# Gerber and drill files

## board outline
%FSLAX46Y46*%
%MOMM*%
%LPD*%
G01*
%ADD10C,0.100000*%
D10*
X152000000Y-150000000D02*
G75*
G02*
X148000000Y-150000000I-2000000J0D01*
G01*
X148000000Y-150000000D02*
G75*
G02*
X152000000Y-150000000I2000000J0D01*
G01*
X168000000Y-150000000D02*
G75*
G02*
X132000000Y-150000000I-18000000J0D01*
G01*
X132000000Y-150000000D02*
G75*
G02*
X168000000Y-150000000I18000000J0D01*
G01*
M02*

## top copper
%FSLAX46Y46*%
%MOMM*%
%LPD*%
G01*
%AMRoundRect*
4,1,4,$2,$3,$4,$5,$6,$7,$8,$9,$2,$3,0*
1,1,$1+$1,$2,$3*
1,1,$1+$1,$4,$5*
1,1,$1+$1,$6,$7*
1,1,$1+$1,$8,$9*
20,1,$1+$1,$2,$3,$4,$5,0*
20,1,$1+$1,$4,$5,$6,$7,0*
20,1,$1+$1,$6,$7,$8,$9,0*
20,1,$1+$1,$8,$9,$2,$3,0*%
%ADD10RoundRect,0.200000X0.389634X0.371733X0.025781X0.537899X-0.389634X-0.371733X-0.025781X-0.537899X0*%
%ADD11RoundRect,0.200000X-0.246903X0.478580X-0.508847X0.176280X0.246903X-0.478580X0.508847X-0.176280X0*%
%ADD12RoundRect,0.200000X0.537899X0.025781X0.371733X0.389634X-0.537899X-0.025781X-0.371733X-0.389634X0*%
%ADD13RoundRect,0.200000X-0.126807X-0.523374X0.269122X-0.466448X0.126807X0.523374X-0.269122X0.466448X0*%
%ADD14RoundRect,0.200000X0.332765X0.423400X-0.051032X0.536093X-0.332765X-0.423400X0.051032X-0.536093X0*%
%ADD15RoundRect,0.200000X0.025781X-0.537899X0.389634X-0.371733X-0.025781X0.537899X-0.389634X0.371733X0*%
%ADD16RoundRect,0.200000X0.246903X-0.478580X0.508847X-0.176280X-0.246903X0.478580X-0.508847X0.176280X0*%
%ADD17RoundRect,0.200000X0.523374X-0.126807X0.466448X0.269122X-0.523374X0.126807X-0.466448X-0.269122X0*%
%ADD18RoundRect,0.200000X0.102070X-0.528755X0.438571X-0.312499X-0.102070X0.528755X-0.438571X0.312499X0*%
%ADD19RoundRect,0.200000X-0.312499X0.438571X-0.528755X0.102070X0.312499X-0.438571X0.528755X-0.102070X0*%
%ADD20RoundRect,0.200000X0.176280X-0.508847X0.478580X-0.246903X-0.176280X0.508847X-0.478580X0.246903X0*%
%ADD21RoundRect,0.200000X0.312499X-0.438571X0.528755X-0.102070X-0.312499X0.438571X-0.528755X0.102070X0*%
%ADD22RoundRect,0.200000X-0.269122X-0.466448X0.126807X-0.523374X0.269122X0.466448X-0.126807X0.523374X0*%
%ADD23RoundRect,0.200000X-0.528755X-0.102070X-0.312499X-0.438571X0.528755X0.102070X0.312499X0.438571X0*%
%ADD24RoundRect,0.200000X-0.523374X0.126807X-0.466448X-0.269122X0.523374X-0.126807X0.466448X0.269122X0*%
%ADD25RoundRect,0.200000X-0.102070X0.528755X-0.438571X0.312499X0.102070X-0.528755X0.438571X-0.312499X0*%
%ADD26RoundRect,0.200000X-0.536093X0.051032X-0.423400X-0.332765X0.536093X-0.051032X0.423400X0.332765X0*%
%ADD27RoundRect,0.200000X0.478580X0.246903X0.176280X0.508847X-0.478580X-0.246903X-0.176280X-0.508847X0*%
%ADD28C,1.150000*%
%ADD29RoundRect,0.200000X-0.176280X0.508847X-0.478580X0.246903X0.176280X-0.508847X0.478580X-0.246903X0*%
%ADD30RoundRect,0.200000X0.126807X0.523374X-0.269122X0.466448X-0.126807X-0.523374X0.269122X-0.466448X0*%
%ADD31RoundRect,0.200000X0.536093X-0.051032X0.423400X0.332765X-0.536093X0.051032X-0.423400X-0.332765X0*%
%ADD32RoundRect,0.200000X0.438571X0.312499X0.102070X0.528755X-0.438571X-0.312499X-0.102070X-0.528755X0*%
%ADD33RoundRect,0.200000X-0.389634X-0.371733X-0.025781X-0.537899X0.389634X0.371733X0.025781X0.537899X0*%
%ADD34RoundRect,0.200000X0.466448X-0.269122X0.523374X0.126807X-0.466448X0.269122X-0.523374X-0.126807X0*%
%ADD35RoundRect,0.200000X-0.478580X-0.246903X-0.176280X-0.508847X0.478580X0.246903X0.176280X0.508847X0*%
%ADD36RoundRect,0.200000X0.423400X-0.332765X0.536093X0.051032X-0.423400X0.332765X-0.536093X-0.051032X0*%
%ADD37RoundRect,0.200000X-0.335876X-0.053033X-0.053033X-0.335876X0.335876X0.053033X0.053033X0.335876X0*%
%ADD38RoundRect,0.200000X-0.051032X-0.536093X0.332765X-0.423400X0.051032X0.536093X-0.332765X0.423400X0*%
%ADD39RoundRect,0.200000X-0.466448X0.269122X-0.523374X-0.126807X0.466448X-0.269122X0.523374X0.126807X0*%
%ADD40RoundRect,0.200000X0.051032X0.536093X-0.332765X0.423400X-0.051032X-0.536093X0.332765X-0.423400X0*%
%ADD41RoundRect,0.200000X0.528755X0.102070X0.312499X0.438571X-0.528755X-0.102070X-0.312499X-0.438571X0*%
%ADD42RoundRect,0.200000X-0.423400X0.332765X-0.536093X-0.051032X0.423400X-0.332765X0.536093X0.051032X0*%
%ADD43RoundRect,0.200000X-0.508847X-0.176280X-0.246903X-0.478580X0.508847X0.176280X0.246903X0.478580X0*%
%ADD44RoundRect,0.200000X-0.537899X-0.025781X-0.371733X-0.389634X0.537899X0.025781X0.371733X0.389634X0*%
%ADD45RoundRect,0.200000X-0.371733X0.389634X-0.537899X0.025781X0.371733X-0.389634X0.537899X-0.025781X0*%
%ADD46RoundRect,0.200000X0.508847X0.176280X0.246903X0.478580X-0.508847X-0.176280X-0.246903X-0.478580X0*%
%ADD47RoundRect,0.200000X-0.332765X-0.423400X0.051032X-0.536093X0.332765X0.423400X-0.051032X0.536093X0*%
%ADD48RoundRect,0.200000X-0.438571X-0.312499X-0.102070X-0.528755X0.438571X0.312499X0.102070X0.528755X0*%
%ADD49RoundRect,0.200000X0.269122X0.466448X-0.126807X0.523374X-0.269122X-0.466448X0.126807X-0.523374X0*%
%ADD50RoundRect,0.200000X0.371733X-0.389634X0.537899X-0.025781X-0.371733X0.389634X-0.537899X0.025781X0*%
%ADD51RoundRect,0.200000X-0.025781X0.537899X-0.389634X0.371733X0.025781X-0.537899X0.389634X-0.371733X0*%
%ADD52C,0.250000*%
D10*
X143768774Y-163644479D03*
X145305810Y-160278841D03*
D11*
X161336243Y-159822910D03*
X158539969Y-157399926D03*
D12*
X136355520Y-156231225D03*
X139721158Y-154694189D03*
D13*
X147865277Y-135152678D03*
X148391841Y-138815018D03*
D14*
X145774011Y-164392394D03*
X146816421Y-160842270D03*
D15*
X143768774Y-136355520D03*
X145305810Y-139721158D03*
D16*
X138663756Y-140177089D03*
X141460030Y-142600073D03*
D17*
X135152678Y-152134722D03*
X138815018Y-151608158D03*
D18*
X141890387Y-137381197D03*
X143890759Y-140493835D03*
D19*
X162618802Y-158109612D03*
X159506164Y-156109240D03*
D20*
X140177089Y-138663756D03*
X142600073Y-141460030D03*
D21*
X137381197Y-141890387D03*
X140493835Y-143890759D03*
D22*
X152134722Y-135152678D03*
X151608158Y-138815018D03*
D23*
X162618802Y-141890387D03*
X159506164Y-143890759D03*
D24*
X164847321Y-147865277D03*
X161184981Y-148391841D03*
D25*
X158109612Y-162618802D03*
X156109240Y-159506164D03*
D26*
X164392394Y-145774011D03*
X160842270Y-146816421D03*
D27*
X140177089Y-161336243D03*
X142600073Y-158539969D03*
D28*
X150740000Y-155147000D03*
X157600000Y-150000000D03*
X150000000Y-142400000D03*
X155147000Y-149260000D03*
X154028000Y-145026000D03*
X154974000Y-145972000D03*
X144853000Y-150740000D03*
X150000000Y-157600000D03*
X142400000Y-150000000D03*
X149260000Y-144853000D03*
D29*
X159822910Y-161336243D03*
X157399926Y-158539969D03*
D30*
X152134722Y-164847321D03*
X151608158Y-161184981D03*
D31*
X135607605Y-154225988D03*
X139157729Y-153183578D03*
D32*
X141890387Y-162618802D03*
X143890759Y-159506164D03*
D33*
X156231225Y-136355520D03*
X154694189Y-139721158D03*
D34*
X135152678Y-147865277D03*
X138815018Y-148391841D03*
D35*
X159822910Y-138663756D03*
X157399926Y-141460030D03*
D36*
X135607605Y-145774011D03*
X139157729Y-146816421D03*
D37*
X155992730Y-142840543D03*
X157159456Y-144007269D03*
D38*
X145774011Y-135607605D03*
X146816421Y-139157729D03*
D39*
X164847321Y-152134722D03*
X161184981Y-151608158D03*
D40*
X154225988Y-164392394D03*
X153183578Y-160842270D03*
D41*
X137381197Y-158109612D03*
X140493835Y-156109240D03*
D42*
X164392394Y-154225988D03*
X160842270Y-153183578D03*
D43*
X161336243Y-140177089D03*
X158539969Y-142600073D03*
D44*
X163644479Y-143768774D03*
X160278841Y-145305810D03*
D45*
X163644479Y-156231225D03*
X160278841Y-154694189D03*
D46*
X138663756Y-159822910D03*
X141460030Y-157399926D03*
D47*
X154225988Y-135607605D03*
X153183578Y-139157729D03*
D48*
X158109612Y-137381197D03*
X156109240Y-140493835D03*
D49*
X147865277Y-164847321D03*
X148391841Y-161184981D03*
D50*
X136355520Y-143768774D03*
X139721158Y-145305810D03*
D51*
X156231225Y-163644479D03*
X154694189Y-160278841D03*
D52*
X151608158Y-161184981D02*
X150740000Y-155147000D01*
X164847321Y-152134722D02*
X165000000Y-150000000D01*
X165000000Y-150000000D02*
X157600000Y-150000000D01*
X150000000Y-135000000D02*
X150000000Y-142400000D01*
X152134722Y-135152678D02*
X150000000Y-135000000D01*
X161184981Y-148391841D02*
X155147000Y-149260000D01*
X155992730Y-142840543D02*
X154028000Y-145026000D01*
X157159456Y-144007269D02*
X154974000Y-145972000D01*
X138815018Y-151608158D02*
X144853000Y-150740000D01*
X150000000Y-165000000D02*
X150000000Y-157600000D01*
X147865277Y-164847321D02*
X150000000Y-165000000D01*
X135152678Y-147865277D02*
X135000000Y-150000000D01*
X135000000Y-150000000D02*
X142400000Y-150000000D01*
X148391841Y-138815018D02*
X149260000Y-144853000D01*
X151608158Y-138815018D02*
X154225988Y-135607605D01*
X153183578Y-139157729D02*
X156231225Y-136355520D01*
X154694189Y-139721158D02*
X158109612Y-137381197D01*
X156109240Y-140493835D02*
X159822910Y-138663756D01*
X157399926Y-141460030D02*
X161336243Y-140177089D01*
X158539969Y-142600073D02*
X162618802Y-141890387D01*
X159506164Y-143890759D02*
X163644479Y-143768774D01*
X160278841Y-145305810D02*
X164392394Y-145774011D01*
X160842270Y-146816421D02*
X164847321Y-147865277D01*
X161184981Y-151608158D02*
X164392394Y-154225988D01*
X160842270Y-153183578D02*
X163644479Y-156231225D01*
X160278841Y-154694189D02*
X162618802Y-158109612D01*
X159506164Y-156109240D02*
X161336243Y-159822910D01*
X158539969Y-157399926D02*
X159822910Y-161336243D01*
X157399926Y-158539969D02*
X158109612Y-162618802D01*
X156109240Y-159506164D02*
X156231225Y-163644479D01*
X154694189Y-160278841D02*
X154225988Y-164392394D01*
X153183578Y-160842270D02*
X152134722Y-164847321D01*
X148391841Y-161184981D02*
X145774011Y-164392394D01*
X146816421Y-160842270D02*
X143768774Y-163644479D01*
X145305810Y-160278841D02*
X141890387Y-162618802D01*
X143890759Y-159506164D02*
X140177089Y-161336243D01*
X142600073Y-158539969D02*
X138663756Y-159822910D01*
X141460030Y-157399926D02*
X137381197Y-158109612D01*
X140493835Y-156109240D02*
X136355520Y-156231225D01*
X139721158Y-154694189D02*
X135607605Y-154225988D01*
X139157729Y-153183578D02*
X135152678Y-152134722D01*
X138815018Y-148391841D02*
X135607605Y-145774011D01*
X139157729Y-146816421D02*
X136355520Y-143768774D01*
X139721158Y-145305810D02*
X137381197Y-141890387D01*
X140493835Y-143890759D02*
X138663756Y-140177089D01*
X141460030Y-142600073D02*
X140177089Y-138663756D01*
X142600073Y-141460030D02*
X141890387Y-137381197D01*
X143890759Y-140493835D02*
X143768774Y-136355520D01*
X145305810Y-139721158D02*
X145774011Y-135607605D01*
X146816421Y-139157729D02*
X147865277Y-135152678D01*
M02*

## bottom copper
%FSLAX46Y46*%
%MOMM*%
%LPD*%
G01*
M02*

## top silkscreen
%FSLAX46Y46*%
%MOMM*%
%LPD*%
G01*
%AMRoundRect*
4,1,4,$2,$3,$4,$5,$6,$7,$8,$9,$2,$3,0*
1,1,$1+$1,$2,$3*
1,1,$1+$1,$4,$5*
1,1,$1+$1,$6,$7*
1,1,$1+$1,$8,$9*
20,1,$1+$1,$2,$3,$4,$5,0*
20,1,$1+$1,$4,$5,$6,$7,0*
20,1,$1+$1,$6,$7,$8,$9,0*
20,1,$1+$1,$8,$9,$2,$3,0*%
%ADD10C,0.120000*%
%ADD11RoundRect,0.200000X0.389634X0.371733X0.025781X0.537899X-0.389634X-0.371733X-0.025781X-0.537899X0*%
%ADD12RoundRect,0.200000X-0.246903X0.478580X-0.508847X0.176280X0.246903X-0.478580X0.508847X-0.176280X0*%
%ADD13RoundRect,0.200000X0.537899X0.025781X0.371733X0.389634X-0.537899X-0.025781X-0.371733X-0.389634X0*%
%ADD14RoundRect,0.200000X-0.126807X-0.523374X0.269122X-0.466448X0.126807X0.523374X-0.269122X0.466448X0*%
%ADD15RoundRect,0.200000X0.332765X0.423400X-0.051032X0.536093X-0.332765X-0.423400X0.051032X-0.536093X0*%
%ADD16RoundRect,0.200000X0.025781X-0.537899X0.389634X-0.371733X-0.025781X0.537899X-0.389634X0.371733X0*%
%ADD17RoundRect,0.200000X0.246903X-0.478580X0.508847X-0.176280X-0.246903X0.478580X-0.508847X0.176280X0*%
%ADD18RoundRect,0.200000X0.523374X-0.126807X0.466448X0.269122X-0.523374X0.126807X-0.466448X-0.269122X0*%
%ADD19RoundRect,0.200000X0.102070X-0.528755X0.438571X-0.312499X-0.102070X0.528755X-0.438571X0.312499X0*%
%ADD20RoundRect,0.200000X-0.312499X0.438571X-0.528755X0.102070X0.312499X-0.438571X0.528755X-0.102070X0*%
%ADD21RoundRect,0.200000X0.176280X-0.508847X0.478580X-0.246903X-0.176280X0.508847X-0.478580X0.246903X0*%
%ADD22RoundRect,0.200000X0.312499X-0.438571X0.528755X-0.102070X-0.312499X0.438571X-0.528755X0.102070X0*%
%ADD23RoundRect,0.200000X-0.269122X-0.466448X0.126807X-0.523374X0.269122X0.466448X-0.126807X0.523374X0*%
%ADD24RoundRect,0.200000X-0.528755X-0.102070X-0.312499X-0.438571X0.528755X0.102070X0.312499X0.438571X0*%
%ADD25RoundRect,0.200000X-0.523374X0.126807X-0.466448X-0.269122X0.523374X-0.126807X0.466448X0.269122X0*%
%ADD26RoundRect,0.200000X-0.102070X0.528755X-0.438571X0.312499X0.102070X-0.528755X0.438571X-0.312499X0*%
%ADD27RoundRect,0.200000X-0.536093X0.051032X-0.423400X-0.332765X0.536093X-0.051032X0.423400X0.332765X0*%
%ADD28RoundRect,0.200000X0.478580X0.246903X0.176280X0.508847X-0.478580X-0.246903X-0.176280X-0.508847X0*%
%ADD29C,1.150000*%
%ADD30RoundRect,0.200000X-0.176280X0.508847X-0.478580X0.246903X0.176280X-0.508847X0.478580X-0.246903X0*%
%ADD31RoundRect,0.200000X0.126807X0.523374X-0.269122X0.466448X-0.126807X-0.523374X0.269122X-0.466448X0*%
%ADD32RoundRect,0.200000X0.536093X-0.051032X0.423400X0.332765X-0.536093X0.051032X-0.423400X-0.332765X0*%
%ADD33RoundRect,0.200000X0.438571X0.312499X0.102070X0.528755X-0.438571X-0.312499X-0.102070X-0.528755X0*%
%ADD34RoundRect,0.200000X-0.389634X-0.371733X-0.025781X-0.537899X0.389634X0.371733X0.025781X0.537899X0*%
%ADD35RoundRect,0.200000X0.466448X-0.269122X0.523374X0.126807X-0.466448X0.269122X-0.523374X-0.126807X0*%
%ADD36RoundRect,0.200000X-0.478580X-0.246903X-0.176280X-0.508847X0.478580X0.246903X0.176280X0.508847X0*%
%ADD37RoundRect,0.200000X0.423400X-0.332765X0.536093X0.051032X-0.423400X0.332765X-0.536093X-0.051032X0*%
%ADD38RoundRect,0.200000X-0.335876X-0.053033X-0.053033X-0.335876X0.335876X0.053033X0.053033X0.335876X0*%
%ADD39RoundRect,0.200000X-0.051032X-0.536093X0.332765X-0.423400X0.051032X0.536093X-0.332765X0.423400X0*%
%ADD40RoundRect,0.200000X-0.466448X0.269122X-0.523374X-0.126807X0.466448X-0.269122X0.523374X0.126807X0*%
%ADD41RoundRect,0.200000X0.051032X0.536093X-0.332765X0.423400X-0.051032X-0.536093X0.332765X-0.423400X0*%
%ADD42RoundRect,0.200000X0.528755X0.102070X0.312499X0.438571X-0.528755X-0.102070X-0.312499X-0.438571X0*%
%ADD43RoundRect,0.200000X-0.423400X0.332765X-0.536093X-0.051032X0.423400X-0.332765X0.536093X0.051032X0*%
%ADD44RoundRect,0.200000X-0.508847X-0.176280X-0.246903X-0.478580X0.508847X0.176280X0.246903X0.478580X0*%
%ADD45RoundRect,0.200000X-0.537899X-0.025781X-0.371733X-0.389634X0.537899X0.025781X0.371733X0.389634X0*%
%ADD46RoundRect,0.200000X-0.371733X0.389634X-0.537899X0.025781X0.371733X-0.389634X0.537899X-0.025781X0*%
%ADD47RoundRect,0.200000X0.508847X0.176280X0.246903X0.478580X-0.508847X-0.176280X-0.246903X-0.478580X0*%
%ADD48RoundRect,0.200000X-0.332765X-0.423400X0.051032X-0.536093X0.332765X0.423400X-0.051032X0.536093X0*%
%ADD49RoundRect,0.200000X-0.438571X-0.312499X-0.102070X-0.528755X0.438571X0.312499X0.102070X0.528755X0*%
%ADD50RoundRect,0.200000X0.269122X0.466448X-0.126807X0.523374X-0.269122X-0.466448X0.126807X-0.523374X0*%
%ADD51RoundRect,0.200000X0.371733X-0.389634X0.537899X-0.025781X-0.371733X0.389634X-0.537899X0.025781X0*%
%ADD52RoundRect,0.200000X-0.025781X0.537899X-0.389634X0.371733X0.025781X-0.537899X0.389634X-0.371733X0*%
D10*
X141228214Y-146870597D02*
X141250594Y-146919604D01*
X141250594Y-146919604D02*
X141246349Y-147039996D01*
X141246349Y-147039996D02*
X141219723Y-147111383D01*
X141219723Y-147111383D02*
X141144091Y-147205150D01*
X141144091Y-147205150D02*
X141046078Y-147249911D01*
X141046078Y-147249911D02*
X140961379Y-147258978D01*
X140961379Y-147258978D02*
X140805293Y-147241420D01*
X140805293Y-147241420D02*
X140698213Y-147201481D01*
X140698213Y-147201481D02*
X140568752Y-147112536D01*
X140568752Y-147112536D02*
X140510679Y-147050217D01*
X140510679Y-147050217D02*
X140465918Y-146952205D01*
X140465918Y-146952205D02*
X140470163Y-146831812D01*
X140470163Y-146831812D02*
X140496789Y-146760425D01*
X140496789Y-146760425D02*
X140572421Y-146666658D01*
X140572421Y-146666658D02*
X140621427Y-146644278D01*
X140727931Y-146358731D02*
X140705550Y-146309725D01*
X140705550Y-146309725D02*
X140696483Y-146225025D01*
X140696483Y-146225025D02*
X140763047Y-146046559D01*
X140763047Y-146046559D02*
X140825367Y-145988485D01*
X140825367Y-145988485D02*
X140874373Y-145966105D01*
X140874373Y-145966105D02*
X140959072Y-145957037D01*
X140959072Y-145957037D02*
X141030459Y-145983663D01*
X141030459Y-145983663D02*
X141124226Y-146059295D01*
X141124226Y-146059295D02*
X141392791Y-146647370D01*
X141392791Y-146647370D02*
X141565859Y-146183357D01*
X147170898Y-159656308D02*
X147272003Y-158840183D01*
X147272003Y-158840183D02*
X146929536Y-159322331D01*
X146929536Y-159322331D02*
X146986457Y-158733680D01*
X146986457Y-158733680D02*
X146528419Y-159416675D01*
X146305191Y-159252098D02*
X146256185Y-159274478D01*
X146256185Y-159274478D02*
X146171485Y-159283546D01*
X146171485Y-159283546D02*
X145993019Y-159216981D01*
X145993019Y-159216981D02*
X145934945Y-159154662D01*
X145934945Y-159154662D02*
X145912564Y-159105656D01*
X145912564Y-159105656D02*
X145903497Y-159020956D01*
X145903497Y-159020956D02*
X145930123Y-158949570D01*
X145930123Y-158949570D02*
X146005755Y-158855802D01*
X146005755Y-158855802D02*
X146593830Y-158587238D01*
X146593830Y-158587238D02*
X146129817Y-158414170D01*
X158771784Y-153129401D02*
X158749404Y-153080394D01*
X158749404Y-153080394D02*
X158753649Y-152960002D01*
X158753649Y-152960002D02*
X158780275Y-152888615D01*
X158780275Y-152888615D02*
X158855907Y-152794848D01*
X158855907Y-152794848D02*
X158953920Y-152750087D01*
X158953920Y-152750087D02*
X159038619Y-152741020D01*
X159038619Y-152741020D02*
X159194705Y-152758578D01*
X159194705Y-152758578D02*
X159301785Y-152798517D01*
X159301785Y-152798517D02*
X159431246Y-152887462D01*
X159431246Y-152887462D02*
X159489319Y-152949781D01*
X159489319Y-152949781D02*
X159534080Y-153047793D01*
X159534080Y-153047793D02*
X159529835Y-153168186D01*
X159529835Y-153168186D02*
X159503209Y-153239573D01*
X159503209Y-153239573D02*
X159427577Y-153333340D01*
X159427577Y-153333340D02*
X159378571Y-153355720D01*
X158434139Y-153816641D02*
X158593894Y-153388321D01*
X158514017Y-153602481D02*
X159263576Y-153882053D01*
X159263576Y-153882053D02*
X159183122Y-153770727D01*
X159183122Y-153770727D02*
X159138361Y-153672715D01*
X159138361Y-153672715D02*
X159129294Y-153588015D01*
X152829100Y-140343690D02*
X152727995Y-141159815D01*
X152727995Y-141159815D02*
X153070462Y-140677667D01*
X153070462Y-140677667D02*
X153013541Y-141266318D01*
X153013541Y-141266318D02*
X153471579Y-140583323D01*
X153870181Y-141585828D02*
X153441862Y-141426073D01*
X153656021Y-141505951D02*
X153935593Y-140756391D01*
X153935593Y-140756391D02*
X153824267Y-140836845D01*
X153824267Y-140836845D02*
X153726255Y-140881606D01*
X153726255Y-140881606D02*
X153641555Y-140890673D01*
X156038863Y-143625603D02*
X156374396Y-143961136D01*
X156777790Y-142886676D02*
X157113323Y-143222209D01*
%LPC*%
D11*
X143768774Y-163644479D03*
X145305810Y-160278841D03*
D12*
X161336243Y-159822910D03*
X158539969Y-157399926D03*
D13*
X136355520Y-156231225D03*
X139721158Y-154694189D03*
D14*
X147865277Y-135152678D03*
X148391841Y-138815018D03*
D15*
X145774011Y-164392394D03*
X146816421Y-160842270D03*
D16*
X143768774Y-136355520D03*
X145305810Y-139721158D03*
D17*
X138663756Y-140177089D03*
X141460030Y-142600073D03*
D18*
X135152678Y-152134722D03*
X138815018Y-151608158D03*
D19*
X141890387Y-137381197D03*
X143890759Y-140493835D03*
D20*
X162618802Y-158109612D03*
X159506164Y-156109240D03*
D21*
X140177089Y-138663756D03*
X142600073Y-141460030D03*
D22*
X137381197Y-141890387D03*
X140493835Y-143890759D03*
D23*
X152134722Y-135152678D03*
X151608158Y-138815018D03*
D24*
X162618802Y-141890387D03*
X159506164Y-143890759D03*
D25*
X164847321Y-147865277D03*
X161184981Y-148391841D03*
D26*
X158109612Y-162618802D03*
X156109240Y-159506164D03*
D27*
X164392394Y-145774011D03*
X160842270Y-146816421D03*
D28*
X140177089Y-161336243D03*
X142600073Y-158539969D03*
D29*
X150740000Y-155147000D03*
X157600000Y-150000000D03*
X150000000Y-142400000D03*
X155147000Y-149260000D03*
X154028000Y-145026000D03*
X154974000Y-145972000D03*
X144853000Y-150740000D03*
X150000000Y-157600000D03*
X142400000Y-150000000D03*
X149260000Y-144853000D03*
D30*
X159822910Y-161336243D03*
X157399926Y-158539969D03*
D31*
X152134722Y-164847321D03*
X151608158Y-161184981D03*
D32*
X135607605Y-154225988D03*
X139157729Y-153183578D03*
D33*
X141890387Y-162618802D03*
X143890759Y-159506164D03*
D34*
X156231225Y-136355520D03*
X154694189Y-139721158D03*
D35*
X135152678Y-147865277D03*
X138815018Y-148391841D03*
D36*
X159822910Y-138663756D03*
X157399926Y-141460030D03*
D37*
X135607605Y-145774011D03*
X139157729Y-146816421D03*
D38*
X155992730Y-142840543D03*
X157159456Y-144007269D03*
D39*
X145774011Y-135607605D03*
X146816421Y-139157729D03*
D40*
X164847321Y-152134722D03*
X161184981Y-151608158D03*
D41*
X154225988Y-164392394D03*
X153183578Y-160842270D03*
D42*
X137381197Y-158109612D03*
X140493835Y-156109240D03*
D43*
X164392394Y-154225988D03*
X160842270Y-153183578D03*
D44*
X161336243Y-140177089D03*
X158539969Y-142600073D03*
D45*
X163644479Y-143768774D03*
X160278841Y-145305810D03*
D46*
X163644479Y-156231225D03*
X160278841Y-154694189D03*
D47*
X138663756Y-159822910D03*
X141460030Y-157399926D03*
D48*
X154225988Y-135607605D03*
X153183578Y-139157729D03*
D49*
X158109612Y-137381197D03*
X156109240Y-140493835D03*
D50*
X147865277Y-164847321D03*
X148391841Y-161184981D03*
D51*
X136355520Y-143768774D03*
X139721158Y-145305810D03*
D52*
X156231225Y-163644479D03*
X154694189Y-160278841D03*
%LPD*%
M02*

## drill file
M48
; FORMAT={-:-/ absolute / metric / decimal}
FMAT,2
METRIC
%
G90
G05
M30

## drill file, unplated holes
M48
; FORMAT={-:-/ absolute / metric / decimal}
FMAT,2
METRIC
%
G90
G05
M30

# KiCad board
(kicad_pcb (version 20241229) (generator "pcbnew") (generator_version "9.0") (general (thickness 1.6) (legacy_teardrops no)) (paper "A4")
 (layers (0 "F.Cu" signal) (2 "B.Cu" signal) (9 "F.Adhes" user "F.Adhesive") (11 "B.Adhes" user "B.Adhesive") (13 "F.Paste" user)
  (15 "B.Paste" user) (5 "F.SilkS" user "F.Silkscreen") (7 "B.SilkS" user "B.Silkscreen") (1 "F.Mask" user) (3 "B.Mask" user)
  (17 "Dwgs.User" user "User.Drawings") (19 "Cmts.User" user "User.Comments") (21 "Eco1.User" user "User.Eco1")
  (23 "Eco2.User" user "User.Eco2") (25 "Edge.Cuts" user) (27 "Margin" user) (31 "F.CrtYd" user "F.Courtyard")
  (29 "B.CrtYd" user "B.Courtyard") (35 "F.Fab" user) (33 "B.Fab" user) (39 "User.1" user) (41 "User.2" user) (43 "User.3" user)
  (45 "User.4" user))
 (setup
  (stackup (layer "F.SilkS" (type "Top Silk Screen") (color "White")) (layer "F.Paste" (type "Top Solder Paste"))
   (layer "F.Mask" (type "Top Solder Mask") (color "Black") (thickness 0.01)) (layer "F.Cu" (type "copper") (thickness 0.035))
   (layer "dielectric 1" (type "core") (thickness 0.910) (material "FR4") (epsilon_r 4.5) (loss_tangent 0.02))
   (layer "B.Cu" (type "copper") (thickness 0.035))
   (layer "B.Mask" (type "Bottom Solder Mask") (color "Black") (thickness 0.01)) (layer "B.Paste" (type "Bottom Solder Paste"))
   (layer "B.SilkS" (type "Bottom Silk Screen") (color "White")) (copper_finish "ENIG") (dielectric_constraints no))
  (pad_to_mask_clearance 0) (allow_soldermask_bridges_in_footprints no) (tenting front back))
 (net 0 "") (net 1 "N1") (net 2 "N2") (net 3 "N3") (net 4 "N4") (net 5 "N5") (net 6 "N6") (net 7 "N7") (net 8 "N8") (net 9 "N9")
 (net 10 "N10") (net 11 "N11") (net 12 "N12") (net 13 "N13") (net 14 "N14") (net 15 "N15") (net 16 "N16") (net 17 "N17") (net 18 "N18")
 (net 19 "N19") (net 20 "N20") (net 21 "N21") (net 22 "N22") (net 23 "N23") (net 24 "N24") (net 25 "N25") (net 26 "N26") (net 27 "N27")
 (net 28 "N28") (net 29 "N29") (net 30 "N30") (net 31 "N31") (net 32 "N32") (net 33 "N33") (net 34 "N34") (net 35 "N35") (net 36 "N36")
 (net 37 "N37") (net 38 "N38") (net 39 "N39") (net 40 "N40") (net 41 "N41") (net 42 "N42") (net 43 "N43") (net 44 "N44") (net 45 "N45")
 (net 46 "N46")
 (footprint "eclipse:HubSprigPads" (layer "F.Cu") (at 144.537292 161.96166 155.4545455)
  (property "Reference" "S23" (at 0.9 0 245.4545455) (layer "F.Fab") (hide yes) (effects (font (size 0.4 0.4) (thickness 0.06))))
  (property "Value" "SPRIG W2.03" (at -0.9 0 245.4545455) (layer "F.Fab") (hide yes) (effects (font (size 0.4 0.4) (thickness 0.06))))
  (pad "1" smd roundrect (at 0 -1.85 155.4545455) (size 0.8 1.4) (layers "F.Cu" "F.Mask") (roundrect_rratio 0.25) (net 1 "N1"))
  (pad "2" smd roundrect (at 0 1.85 155.4545455) (size 0.8 1.4) (layers "F.Cu" "F.Mask") (roundrect_rratio 0.25) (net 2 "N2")))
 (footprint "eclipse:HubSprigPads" (layer "F.Cu") (at 159.938106 158.611418 -130.9090909)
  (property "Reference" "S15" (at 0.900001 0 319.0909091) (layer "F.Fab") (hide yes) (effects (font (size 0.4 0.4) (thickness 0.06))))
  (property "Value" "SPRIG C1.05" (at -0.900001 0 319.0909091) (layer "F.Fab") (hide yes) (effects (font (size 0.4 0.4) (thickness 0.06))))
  (pad "1" smd roundrect (at 0 -1.85 229.0909091) (size 0.8 1.4) (layers "F.Cu" "F.Mask") (roundrect_rratio 0.25) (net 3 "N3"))
  (pad "2" smd roundrect (at 0 1.85 229.0909091) (size 0.8 1.4) (layers "F.Cu" "F.Mask") (roundrect_rratio 0.25) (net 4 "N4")))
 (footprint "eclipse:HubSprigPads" (layer "F.Cu") (at 138.038339 155.462707 114.5454545)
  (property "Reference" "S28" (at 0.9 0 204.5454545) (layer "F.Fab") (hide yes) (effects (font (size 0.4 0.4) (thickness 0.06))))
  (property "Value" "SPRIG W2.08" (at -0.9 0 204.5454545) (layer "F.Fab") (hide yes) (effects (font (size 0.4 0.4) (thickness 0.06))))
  (pad "1" smd roundrect (at 0 -1.85 114.5454545) (size 0.8 1.4) (layers "F.Cu" "F.Mask") (roundrect_rratio 0.25) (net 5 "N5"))
  (pad "2" smd roundrect (at 0 1.85 114.5454545) (size 0.8 1.4) (layers "F.Cu" "F.Mask") (roundrect_rratio 0.25) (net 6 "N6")))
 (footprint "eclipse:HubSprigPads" (layer "F.Cu") (at 148.128559 136.983848 8.181818182)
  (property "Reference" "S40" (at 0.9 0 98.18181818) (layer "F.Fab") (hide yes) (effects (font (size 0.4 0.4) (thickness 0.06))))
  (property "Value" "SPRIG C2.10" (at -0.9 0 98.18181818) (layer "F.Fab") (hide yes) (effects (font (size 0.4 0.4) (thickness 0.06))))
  (pad "1" smd roundrect (at 0 -1.85 8.181818182) (size 0.8 1.4) (layers "F.Cu" "F.Mask") (roundrect_rratio 0.25) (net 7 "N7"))
  (pad "2" smd roundrect (at 0 1.85 8.181818182) (size 0.8 1.4) (layers "F.Cu" "F.Mask") (roundrect_rratio 0.25) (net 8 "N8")))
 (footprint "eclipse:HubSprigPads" (layer "F.Cu") (at 146.295216 162.617332 163.6363636)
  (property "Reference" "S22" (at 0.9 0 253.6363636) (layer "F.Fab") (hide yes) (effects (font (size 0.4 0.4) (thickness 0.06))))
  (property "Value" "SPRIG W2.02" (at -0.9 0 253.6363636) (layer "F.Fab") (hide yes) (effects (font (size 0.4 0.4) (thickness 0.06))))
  (pad "1" smd roundrect (at 0 -1.85 163.6363636) (size 0.8 1.4) (layers "F.Cu" "F.Mask") (roundrect_rratio 0.25) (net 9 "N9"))
  (pad "2" smd roundrect (at 0 1.85 163.6363636) (size 0.8 1.4) (layers "F.Cu" "F.Mask") (roundrect_rratio 0.25) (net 1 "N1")))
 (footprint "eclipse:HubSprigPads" (layer "F.Cu") (at 144.537292 138.038339 24.54545455)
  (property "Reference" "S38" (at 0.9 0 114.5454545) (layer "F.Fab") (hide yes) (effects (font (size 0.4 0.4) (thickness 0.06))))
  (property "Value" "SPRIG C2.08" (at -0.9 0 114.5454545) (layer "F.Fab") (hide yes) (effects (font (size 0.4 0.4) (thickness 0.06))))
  (pad "1" smd roundrect (at 0 -1.85 24.54545455) (size 0.8 1.4) (layers "F.Cu" "F.Mask") (roundrect_rratio 0.25) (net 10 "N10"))
  (pad "2" smd roundrect (at 0 1.85 24.54545455) (size 0.8 1.4) (layers "F.Cu" "F.Mask") (roundrect_rratio 0.25) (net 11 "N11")))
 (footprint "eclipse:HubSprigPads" (layer "F.Cu") (at 140.061893 141.388581 49.09090909)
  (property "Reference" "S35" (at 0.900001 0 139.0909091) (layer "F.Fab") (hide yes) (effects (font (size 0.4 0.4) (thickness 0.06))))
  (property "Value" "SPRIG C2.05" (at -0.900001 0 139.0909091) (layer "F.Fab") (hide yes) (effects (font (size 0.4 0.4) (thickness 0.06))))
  (pad "1" smd roundrect (at 0 -1.85 49.09090909) (size 0.8 1.4) (layers "F.Cu" "F.Mask") (roundrect_rratio 0.25) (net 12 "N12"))
  (pad "2" smd roundrect (at 0 1.85 49.09090909) (size 0.8 1.4) (layers "F.Cu" "F.Mask") (roundrect_rratio 0.25) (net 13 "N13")))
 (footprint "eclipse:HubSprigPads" (layer "F.Cu") (at 136.983848 151.87144 98.18181818)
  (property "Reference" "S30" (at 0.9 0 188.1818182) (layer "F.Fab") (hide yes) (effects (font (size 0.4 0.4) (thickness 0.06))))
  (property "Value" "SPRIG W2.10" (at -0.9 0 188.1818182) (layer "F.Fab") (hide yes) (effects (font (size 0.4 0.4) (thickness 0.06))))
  (pad "1" smd roundrect (at 0 -1.85 98.18181818) (size 0.8 1.4) (layers "F.Cu" "F.Mask") (roundrect_rratio 0.25) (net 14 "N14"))
  (pad "2" smd roundrect (at 0 1.85 98.18181818) (size 0.8 1.4) (layers "F.Cu" "F.Mask") (roundrect_rratio 0.25) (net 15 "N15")))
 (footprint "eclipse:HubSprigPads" (layer "F.Cu") (at 142.890573 138.937516 32.72727273)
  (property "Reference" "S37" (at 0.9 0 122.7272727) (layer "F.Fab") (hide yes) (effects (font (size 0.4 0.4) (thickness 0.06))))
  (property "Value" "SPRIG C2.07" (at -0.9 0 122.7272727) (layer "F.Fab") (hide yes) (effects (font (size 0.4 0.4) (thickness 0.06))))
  (pad "1" smd roundrect (at 0 -1.85 32.72727273) (size 0.8 1.4) (layers "F.Cu" "F.Mask") (roundrect_rratio 0.25) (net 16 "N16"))
  (pad "2" smd roundrect (at 0 1.85 32.72727273) (size 0.8 1.4) (layers "F.Cu" "F.Mask") (roundrect_rratio 0.25) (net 10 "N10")))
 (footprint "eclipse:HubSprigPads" (layer "F.Cu") (at 161.062483 157.109426 -122.7272727)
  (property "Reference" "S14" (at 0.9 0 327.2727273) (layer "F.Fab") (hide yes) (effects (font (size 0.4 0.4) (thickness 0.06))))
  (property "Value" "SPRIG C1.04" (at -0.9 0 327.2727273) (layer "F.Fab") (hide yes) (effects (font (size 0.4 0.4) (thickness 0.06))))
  (pad "1" smd roundrect (at 0 -1.85 237.2727273) (size 0.8 1.4) (layers "F.Cu" "F.Mask") (roundrect_rratio 0.25) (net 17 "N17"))
  (pad "2" smd roundrect (at 0 1.85 237.2727273) (size 0.8 1.4) (layers "F.Cu" "F.Mask") (roundrect_rratio 0.25) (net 3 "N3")))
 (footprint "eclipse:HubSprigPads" (layer "F.Cu") (at 141.388581 140.061893 40.90909091)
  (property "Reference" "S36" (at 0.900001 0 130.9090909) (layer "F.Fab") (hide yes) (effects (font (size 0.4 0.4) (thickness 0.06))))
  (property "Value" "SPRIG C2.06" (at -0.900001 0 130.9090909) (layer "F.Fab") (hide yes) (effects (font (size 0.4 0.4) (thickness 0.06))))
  (pad "1" smd roundrect (at 0 -1.85 40.90909091) (size 0.8 1.4) (layers "F.Cu" "F.Mask") (roundrect_rratio 0.25) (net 13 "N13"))
  (pad "2" smd roundrect (at 0 1.85 40.90909091) (size 0.8 1.4) (layers "F.Cu" "F.Mask") (roundrect_rratio 0.25) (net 16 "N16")))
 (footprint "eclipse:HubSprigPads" (layer "F.Cu") (at 138.937516 142.890573 57.27272727)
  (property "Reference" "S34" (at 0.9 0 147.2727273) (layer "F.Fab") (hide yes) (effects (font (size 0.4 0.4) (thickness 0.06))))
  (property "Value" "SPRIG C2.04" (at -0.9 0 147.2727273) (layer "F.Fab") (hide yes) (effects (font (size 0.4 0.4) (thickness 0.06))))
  (pad "1" smd roundrect (at 0 -1.85 57.27272727) (size 0.8 1.4) (layers "F.Cu" "F.Mask") (roundrect_rratio 0.25) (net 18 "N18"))
  (pad "2" smd roundrect (at 0 1.85 57.27272727) (size 0.8 1.4) (layers "F.Cu" "F.Mask") (roundrect_rratio 0.25) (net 12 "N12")))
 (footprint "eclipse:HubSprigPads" (layer "F.Cu") (at 151.87144 136.983848 -8.181818182)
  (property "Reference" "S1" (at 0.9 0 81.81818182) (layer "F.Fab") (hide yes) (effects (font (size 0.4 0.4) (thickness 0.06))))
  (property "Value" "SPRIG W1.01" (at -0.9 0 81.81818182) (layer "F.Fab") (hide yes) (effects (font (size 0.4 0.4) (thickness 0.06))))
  (pad "1" smd roundrect (at 0 -1.85 351.8181818) (size 0.8 1.4) (layers "F.Cu" "F.Mask") (roundrect_rratio 0.25) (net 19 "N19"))
  (pad "2" smd roundrect (at 0 1.85 351.8181818) (size 0.8 1.4) (layers "F.Cu" "F.Mask") (roundrect_rratio 0.25) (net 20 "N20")))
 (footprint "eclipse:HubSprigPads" (layer "F.Cu") (at 161.062483 142.890573 -57.27272727)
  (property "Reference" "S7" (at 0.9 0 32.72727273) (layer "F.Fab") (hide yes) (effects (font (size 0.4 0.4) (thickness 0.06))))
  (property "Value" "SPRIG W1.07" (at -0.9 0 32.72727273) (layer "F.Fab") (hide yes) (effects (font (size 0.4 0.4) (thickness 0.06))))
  (pad "1" smd roundrect (at 0 -1.85 302.7272727) (size 0.8 1.4) (layers "F.Cu" "F.Mask") (roundrect_rratio 0.25) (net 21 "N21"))
  (pad "2" smd roundrect (at 0 1.85 302.7272727) (size 0.8 1.4) (layers "F.Cu" "F.Mask") (roundrect_rratio 0.25) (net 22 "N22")))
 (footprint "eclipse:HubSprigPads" (layer "F.Cu") (at 163.016151 148.128559 -81.81818182)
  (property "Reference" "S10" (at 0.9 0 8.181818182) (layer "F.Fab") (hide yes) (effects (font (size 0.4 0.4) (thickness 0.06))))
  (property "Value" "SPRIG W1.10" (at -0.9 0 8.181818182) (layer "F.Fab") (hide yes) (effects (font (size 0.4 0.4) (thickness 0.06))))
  (pad "1" smd roundrect (at 0 -1.85 278.1818182) (size 0.8 1.4) (layers "F.Cu" "F.Mask") (roundrect_rratio 0.25) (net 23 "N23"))
  (pad "2" smd roundrect (at 0 1.85 278.1818182) (size 0.8 1.4) (layers "F.Cu" "F.Mask") (roundrect_rratio 0.25) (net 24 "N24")))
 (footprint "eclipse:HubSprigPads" (layer "F.Cu") (at 157.109426 161.062483 -147.2727273)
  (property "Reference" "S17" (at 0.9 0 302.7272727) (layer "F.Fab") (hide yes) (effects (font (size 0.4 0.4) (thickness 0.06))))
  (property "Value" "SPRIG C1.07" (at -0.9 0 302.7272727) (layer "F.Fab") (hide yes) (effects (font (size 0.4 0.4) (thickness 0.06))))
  (pad "1" smd roundrect (at 0 -1.85 212.7272727) (size 0.8 1.4) (layers "F.Cu" "F.Mask") (roundrect_rratio 0.25) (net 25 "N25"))
  (pad "2" smd roundrect (at 0 1.85 212.7272727) (size 0.8 1.4) (layers "F.Cu" "F.Mask") (roundrect_rratio 0.25) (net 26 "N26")))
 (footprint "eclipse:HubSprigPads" (layer "F.Cu") (at 162.617332 146.295216 -73.63636364)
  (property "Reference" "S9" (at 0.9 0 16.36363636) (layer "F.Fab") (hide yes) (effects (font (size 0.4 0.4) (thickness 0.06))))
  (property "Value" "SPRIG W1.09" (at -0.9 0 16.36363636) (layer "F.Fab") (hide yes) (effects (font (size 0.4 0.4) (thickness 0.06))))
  (pad "1" smd roundrect (at 0 -1.85 286.3636364) (size 0.8 1.4) (layers "F.Cu" "F.Mask") (roundrect_rratio 0.25) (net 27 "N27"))
  (pad "2" smd roundrect (at 0 1.85 286.3636364) (size 0.8 1.4) (layers "F.Cu" "F.Mask") (roundrect_rratio 0.25) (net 23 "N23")))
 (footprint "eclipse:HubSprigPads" (layer "F.Cu") (at 141.388581 159.938106 139.0909091)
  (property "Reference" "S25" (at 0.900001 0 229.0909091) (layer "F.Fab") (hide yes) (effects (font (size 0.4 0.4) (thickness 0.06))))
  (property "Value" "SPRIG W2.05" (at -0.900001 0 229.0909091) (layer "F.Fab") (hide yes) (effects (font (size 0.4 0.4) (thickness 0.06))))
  (pad "1" smd roundrect (at 0 -1.85 139.0909091) (size 0.8 1.4) (layers "F.Cu" "F.Mask") (roundrect_rratio 0.25) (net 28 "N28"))
  (pad "2" smd roundrect (at 0 1.85 139.0909091) (size 0.8 1.4) (layers "F.Cu" "F.Mask") (roundrect_rratio 0.25) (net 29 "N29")))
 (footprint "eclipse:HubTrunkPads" (layer "F.Cu") (at 150 150)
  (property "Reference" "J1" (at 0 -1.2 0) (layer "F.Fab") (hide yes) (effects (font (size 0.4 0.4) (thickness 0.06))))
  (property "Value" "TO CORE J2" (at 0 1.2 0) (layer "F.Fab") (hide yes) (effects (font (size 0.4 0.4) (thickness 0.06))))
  (pad "1" smd circle (at 0.74 5.147) (size 1.15 1.15) (layers "F.Cu" "F.Mask") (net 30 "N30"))
  (pad "2" smd circle (at 7.6 0) (size 1.15 1.15) (layers "F.Cu" "F.Mask") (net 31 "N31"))
  (pad "3" smd circle (at 0 -7.6) (size 1.15 1.15) (layers "F.Cu" "F.Mask") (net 19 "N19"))
  (pad "4" smd circle (at 5.147 -0.74) (size 1.15 1.15) (layers "F.Cu" "F.Mask") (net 24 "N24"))
  (pad "5" smd circle (at 4.028 -4.974) (size 1.15 1.15) (layers "F.Cu" "F.Mask") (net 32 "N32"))
  (pad "6" smd circle (at 4.974 -4.028) (size 1.15 1.15) (layers "F.Cu" "F.Mask") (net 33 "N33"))
  (pad "7" smd circle (at -5.147 0.74) (size 1.15 1.15) (layers "F.Cu" "F.Mask") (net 15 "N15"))
  (pad "8" smd circle (at 0 7.6) (size 1.15 1.15) (layers "F.Cu" "F.Mask") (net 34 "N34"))
  (pad "9" smd circle (at -7.6 0) (size 1.15 1.15) (layers "F.Cu" "F.Mask") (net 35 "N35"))
  (pad "10" smd circle (at -0.74 -5.147) (size 1.15 1.15) (layers "F.Cu" "F.Mask") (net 8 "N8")))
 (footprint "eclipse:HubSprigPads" (layer "F.Cu") (at 158.611418 159.938106 -139.0909091)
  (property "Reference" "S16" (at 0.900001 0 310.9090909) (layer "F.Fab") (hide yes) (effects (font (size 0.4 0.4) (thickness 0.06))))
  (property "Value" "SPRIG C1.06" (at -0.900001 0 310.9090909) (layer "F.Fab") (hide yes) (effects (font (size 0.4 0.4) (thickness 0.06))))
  (pad "1" smd roundrect (at 0 -1.85 220.9090909) (size 0.8 1.4) (layers "F.Cu" "F.Mask") (roundrect_rratio 0.25) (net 4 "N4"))
  (pad "2" smd roundrect (at 0 1.85 220.9090909) (size 0.8 1.4) (layers "F.Cu" "F.Mask") (roundrect_rratio 0.25) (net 25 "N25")))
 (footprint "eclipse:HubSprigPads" (layer "F.Cu") (at 151.87144 163.016151 -171.8181818)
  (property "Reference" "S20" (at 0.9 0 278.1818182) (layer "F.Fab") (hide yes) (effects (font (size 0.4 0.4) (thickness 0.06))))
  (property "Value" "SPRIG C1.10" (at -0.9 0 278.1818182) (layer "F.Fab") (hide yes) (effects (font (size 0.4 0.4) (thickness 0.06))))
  (pad "1" smd roundrect (at 0 -1.85 188.1818182) (size 0.8 1.4) (layers "F.Cu" "F.Mask") (roundrect_rratio 0.25) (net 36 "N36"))
  (pad "2" smd roundrect (at 0 1.85 188.1818182) (size 0.8 1.4) (layers "F.Cu" "F.Mask") (roundrect_rratio 0.25) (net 30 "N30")))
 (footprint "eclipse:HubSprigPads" (layer "F.Cu") (at 137.382667 153.704783 106.3636364)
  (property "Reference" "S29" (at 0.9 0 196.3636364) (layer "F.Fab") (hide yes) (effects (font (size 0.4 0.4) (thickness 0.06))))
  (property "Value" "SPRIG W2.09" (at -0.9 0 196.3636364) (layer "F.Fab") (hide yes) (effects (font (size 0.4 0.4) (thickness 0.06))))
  (pad "1" smd roundrect (at 0 -1.85 106.3636364) (size 0.8 1.4) (layers "F.Cu" "F.Mask") (roundrect_rratio 0.25) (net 6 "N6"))
  (pad "2" smd roundrect (at 0 1.85 106.3636364) (size 0.8 1.4) (layers "F.Cu" "F.Mask") (roundrect_rratio 0.25) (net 14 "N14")))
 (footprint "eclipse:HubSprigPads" (layer "F.Cu") (at 142.890573 161.062483 147.2727273)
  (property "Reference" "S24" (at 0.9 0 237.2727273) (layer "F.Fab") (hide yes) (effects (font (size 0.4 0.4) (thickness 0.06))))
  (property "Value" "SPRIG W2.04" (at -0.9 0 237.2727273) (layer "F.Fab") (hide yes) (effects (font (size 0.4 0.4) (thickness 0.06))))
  (pad "1" smd roundrect (at 0 -1.85 147.2727273) (size 0.8 1.4) (layers "F.Cu" "F.Mask") (roundrect_rratio 0.25) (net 2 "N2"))
  (pad "2" smd roundrect (at 0 1.85 147.2727273) (size 0.8 1.4) (layers "F.Cu" "F.Mask") (roundrect_rratio 0.25) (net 28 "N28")))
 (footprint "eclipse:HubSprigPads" (layer "F.Cu") (at 155.462707 138.038339 -24.54545455)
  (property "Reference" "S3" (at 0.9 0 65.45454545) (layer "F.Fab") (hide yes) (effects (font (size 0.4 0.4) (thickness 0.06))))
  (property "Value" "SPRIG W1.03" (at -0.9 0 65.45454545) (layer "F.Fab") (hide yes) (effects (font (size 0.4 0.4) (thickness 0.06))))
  (pad "1" smd roundrect (at 0 -1.85 335.4545455) (size 0.8 1.4) (layers "F.Cu" "F.Mask") (roundrect_rratio 0.25) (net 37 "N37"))
  (pad "2" smd roundrect (at 0 1.85 335.4545455) (size 0.8 1.4) (layers "F.Cu" "F.Mask") (roundrect_rratio 0.25) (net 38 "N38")))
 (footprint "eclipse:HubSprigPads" (layer "F.Cu") (at 136.983848 148.128559 81.81818182)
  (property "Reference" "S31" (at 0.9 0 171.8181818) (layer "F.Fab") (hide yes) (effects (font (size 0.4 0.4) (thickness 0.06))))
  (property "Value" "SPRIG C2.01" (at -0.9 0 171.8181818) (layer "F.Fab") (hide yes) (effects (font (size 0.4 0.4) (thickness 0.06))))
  (pad "1" smd roundrect (at 0 -1.85 81.81818182) (size 0.8 1.4) (layers "F.Cu" "F.Mask") (roundrect_rratio 0.25) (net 35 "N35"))
  (pad "2" smd roundrect (at 0 1.85 81.81818182) (size 0.8 1.4) (layers "F.Cu" "F.Mask") (roundrect_rratio 0.25) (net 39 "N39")))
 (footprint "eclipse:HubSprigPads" (layer "F.Cu") (at 158.611418 140.061893 -40.90909091)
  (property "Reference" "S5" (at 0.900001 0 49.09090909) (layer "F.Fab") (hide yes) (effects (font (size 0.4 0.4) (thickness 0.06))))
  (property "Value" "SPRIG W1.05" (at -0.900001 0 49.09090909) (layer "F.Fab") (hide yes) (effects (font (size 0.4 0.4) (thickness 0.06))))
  (pad "1" smd roundrect (at 0 -1.85 319.0909091) (size 0.8 1.4) (layers "F.Cu" "F.Mask") (roundrect_rratio 0.25) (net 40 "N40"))
  (pad "2" smd roundrect (at 0 1.85 319.0909091) (size 0.8 1.4) (layers "F.Cu" "F.Mask") (roundrect_rratio 0.25) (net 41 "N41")))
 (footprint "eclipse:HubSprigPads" (layer "F.Cu") (at 137.382667 146.295216 73.63636364)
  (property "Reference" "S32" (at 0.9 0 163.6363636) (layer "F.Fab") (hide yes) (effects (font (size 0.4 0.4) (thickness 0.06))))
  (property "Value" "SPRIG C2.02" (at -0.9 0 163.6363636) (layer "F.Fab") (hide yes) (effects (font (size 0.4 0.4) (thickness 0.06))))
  (pad "1" smd roundrect (at 0 -1.85 73.63636364) (size 0.8 1.4) (layers "F.Cu" "F.Mask") (roundrect_rratio 0.25) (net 39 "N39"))
  (pad "2" smd roundrect (at 0 1.85 73.63636364) (size 0.8 1.4) (layers "F.Cu" "F.Mask") (roundrect_rratio 0.25) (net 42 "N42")))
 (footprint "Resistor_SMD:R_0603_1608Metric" (layer "F.Cu") (at 156.576093 143.423906 -45)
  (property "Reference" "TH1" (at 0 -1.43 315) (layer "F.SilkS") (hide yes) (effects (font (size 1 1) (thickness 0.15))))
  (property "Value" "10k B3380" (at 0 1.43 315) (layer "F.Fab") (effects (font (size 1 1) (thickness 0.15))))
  (fp_line (start -0.237258 0.5225) (end 0.237258 0.5225) (stroke (width 0.12) (type solid)) (layer "F.SilkS"))
  (fp_line (start -0.237258 -0.5225) (end 0.237258 -0.5225) (stroke (width 0.12) (type solid)) (layer "F.SilkS"))
  (pad "1" smd roundrect (at -0.825 0 315) (size 0.8 0.95) (layers "F.Cu" "F.Mask" "F.Paste") (roundrect_rratio 0.25) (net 32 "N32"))
  (pad "2" smd roundrect (at 0.825 0 315) (size 0.8 0.95) (layers "F.Cu" "F.Mask" "F.Paste") (roundrect_rratio 0.25) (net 33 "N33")))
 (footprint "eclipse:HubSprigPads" (layer "F.Cu") (at 146.295216 137.382667 16.36363636)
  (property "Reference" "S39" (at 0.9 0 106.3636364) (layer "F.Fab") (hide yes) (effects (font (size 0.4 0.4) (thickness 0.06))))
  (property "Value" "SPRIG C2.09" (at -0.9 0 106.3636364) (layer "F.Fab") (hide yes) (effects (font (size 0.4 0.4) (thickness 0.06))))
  (pad "1" smd roundrect (at 0 -1.85 16.36363636) (size 0.8 1.4) (layers "F.Cu" "F.Mask") (roundrect_rratio 0.25) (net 11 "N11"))
  (pad "2" smd roundrect (at 0 1.85 16.36363636) (size 0.8 1.4) (layers "F.Cu" "F.Mask") (roundrect_rratio 0.25) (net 7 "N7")))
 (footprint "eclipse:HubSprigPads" (layer "F.Cu") (at 163.016151 151.87144 -98.18181818)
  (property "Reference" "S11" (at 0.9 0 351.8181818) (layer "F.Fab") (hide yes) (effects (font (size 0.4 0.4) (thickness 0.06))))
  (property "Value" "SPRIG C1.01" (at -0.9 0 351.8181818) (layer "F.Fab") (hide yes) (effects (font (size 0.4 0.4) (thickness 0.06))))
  (pad "1" smd roundrect (at 0 -1.85 261.8181818) (size 0.8 1.4) (layers "F.Cu" "F.Mask") (roundrect_rratio 0.25) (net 31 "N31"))
  (pad "2" smd roundrect (at 0 1.85 261.8181818) (size 0.8 1.4) (layers "F.Cu" "F.Mask") (roundrect_rratio 0.25) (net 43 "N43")))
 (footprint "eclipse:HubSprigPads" (layer "F.Cu") (at 153.704783 162.617332 -163.6363636)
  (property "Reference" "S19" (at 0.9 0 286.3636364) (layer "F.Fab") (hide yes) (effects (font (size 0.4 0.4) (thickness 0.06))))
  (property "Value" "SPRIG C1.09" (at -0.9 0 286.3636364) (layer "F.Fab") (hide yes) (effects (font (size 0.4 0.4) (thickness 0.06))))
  (pad "1" smd roundrect (at 0 -1.85 196.3636364) (size 0.8 1.4) (layers "F.Cu" "F.Mask") (roundrect_rratio 0.25) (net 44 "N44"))
  (pad "2" smd roundrect (at 0 1.85 196.3636364) (size 0.8 1.4) (layers "F.Cu" "F.Mask") (roundrect_rratio 0.25) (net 36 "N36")))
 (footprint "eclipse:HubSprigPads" (layer "F.Cu") (at 138.937516 157.109426 122.7272727)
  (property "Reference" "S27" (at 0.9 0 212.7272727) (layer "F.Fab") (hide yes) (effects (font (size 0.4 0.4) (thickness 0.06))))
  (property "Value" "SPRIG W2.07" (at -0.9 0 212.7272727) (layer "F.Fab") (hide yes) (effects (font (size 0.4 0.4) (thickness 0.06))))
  (pad "1" smd roundrect (at 0 -1.85 122.7272727) (size 0.8 1.4) (layers "F.Cu" "F.Mask") (roundrect_rratio 0.25) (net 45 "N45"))
  (pad "2" smd roundrect (at 0 1.85 122.7272727) (size 0.8 1.4) (layers "F.Cu" "F.Mask") (roundrect_rratio 0.25) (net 5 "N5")))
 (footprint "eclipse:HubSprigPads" (layer "F.Cu") (at 162.617332 153.704783 -106.3636364)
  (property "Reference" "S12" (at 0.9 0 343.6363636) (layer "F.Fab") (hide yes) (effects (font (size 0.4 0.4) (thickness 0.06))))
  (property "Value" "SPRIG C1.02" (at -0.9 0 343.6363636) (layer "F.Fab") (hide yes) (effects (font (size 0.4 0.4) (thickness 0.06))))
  (pad "1" smd roundrect (at 0 -1.85 253.6363636) (size 0.8 1.4) (layers "F.Cu" "F.Mask") (roundrect_rratio 0.25) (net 43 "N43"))
  (pad "2" smd roundrect (at 0 1.85 253.6363636) (size 0.8 1.4) (layers "F.Cu" "F.Mask") (roundrect_rratio 0.25) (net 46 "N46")))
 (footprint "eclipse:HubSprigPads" (layer "F.Cu") (at 159.938106 141.388581 -49.09090909)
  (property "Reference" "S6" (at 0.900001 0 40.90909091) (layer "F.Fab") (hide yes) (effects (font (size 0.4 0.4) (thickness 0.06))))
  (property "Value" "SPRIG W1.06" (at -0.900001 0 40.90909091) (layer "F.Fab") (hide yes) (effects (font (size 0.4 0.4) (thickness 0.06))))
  (pad "1" smd roundrect (at 0 -1.85 310.9090909) (size 0.8 1.4) (layers "F.Cu" "F.Mask") (roundrect_rratio 0.25) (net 41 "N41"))
  (pad "2" smd roundrect (at 0 1.85 310.9090909) (size 0.8 1.4) (layers "F.Cu" "F.Mask") (roundrect_rratio 0.25) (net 21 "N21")))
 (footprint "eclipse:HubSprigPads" (layer "F.Cu") (at 161.96166 144.537292 -65.45454545)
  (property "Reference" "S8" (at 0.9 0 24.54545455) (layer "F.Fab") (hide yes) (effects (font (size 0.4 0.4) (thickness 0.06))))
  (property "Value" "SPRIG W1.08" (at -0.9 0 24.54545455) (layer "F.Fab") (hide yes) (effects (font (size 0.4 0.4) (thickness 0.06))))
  (pad "1" smd roundrect (at 0 -1.85 294.5454545) (size 0.8 1.4) (layers "F.Cu" "F.Mask") (roundrect_rratio 0.25) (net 22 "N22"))
  (pad "2" smd roundrect (at 0 1.85 294.5454545) (size 0.8 1.4) (layers "F.Cu" "F.Mask") (roundrect_rratio 0.25) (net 27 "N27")))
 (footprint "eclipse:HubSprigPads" (layer "F.Cu") (at 161.96166 155.462707 -114.5454545)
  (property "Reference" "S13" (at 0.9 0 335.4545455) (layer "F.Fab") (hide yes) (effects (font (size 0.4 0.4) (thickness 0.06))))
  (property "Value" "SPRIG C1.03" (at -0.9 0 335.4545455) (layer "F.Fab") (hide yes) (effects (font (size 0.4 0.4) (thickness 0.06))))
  (pad "1" smd roundrect (at 0 -1.85 245.4545455) (size 0.8 1.4) (layers "F.Cu" "F.Mask") (roundrect_rratio 0.25) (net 46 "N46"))
  (pad "2" smd roundrect (at 0 1.85 245.4545455) (size 0.8 1.4) (layers "F.Cu" "F.Mask") (roundrect_rratio 0.25) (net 17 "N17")))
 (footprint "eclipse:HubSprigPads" (layer "F.Cu") (at 140.061893 158.611418 130.9090909)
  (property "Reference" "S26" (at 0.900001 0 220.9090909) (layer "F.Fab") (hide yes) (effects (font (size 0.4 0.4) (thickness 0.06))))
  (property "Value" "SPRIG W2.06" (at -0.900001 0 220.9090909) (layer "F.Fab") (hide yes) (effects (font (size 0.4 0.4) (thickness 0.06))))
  (pad "1" smd roundrect (at 0 -1.85 130.9090909) (size 0.8 1.4) (layers "F.Cu" "F.Mask") (roundrect_rratio 0.25) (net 29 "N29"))
  (pad "2" smd roundrect (at 0 1.85 130.9090909) (size 0.8 1.4) (layers "F.Cu" "F.Mask") (roundrect_rratio 0.25) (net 45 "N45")))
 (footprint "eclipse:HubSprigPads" (layer "F.Cu") (at 153.704783 137.382667 -16.36363636)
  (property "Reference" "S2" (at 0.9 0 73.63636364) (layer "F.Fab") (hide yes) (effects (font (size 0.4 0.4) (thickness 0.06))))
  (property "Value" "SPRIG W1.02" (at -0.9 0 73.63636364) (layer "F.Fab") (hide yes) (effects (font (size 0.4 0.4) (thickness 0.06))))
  (pad "1" smd roundrect (at 0 -1.85 343.6363636) (size 0.8 1.4) (layers "F.Cu" "F.Mask") (roundrect_rratio 0.25) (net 20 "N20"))
  (pad "2" smd roundrect (at 0 1.85 343.6363636) (size 0.8 1.4) (layers "F.Cu" "F.Mask") (roundrect_rratio 0.25) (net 37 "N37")))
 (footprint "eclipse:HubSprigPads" (layer "F.Cu") (at 157.109426 138.937516 -32.72727273)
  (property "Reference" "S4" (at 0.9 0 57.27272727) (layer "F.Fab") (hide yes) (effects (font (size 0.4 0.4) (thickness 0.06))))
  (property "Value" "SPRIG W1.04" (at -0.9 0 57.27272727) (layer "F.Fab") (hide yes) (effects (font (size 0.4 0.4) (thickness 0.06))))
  (pad "1" smd roundrect (at 0 -1.85 327.2727273) (size 0.8 1.4) (layers "F.Cu" "F.Mask") (roundrect_rratio 0.25) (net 38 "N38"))
  (pad "2" smd roundrect (at 0 1.85 327.2727273) (size 0.8 1.4) (layers "F.Cu" "F.Mask") (roundrect_rratio 0.25) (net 40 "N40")))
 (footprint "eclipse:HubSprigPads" (layer "F.Cu") (at 148.128559 163.016151 171.8181818)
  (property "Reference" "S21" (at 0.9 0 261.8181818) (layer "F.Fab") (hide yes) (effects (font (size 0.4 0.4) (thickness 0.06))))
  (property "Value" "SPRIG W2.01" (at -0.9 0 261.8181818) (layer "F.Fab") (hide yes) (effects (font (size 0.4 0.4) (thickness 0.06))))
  (pad "1" smd roundrect (at 0 -1.85 171.8181818) (size 0.8 1.4) (layers "F.Cu" "F.Mask") (roundrect_rratio 0.25) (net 34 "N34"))
  (pad "2" smd roundrect (at 0 1.85 171.8181818) (size 0.8 1.4) (layers "F.Cu" "F.Mask") (roundrect_rratio 0.25) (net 9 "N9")))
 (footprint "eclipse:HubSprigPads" (layer "F.Cu") (at 138.038339 144.537292 65.45454545)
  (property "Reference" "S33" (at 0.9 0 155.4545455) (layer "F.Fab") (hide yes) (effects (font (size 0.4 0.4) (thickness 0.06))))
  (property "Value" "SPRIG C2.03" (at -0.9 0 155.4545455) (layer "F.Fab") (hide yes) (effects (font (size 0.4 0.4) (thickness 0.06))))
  (pad "1" smd roundrect (at 0 -1.85 65.45454545) (size 0.8 1.4) (layers "F.Cu" "F.Mask") (roundrect_rratio 0.25) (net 42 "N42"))
  (pad "2" smd roundrect (at 0 1.85 65.45454545) (size 0.8 1.4) (layers "F.Cu" "F.Mask") (roundrect_rratio 0.25) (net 18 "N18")))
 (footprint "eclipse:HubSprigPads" (layer "F.Cu") (at 155.462707 161.96166 -155.4545455)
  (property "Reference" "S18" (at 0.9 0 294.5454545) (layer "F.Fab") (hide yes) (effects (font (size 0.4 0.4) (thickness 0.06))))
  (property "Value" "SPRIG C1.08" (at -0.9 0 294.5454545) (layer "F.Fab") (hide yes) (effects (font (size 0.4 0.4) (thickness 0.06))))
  (pad "1" smd roundrect (at 0 -1.85 204.5454545) (size 0.8 1.4) (layers "F.Cu" "F.Mask") (roundrect_rratio 0.25) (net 26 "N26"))
  (pad "2" smd roundrect (at 0 1.85 204.5454545) (size 0.8 1.4) (layers "F.Cu" "F.Mask") (roundrect_rratio 0.25) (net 44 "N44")))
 (gr_circle (center 150 150) (end 152 150) (stroke (width 0.1) (type default)) (fill no) (layer "Edge.Cuts"))
 (gr_circle (center 150 150) (end 168 150) (stroke (width 0.1) (type default)) (fill no) (layer "Edge.Cuts"))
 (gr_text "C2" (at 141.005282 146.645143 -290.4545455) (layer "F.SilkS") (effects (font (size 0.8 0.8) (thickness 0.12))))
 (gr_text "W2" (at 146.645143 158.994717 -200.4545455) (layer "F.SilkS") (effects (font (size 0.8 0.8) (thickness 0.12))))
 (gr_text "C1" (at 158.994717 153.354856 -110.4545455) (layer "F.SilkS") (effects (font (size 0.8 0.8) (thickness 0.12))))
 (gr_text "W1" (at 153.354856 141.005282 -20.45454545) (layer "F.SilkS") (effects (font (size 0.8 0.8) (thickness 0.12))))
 (segment (start 151.608158 161.184981) (end 150.74 155.147) (width 0.25) (layer "F.Cu") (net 30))
 (segment (start 164.847321 152.134722) (end 165 150) (width 0.25) (layer "F.Cu") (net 31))
 (segment (start 165 150) (end 157.6 150) (width 0.25) (layer "F.Cu") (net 31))
 (segment (start 150 135) (end 150 142.4) (width 0.25) (layer "F.Cu") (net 19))
 (segment (start 152.134722 135.152678) (end 150 135) (width 0.25) (layer "F.Cu") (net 19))
 (segment (start 161.184981 148.391841) (end 155.147 149.26) (width 0.25) (layer "F.Cu") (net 24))
 (segment (start 155.99273 142.840543) (end 154.028 145.026) (width 0.25) (layer "F.Cu") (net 32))
 (segment (start 157.159456 144.007269) (end 154.974 145.972) (width 0.25) (layer "F.Cu") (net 33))
 (segment (start 138.815018 151.608158) (end 144.853 150.74) (width 0.25) (layer "F.Cu") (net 15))
 (segment (start 150 165) (end 150 157.6) (width 0.25) (layer "F.Cu") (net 34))
 (segment (start 147.865277 164.847321) (end 150 165) (width 0.25) (layer "F.Cu") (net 34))
 (segment (start 135.152678 147.865277) (end 135 150) (width 0.25) (layer "F.Cu") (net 35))
 (segment (start 135 150) (end 142.4 150) (width 0.25) (layer "F.Cu") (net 35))
 (segment (start 148.391841 138.815018) (end 149.26 144.853) (width 0.25) (layer "F.Cu") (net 8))
 (segment (start 151.608158 138.815018) (end 154.225988 135.607605) (width 0.25) (layer "F.Cu") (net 20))
 (segment (start 153.183578 139.157729) (end 156.231225 136.35552) (width 0.25) (layer "F.Cu") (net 37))
 (segment (start 154.694189 139.721158) (end 158.109612 137.381197) (width 0.25) (layer "F.Cu") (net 38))
 (segment (start 156.10924 140.493835) (end 159.82291 138.663756) (width 0.25) (layer "F.Cu") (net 40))
 (segment (start 157.399926 141.46003) (end 161.336243 140.177089) (width 0.25) (layer "F.Cu") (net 41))
 (segment (start 158.539969 142.600073) (end 162.618802 141.890387) (width 0.25) (layer "F.Cu") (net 21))
 (segment (start 159.506164 143.890759) (end 163.644479 143.768774) (width 0.25) (layer "F.Cu") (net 22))
 (segment (start 160.278841 145.30581) (end 164.392394 145.774011) (width 0.25) (layer "F.Cu") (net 27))
 (segment (start 160.84227 146.816421) (end 164.847321 147.865277) (width 0.25) (layer "F.Cu") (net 23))
 (segment (start 161.184981 151.608158) (end 164.392394 154.225988) (width 0.25) (layer "F.Cu") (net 43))
 (segment (start 160.84227 153.183578) (end 163.644479 156.231225) (width 0.25) (layer "F.Cu") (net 46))
 (segment (start 160.278841 154.694189) (end 162.618802 158.109612) (width 0.25) (layer "F.Cu") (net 17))
 (segment (start 159.506164 156.10924) (end 161.336243 159.82291) (width 0.25) (layer "F.Cu") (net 3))
 (segment (start 158.539969 157.399926) (end 159.82291 161.336243) (width 0.25) (layer "F.Cu") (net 4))
 (segment (start 157.399926 158.539969) (end 158.109612 162.618802) (width 0.25) (layer "F.Cu") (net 25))
 (segment (start 156.10924 159.506164) (end 156.231225 163.644479) (width 0.25) (layer "F.Cu") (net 26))
 (segment (start 154.694189 160.278841) (end 154.225988 164.392394) (width 0.25) (layer "F.Cu") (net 44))
 (segment (start 153.183578 160.84227) (end 152.134722 164.847321) (width 0.25) (layer "F.Cu") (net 36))
 (segment (start 148.391841 161.184981) (end 145.774011 164.392394) (width 0.25) (layer "F.Cu") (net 9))
 (segment (start 146.816421 160.84227) (end 143.768774 163.644479) (width 0.25) (layer "F.Cu") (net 1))
 (segment (start 145.30581 160.278841) (end 141.890387 162.618802) (width 0.25) (layer "F.Cu") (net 2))
 (segment (start 143.890759 159.506164) (end 140.177089 161.336243) (width 0.25) (layer "F.Cu") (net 28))
 (segment (start 142.600073 158.539969) (end 138.663756 159.82291) (width 0.25) (layer "F.Cu") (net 29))
 (segment (start 141.46003 157.399926) (end 137.381197 158.109612) (width 0.25) (layer "F.Cu") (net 45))
 (segment (start 140.493835 156.10924) (end 136.35552 156.231225) (width 0.25) (layer "F.Cu") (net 5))
 (segment (start 139.721158 154.694189) (end 135.607605 154.225988) (width 0.25) (layer "F.Cu") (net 6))
 (segment (start 139.157729 153.183578) (end 135.152678 152.134722) (width 0.25) (layer "F.Cu") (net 14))
 (segment (start 138.815018 148.391841) (end 135.607605 145.774011) (width 0.25) (layer "F.Cu") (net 39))
 (segment (start 139.157729 146.816421) (end 136.35552 143.768774) (width 0.25) (layer "F.Cu") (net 42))
 (segment (start 139.721158 145.30581) (end 137.381197 141.890387) (width 0.25) (layer "F.Cu") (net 18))
 (segment (start 140.493835 143.890759) (end 138.663756 140.177089) (width 0.25) (layer "F.Cu") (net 12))
 (segment (start 141.46003 142.600073) (end 140.177089 138.663756) (width 0.25) (layer "F.Cu") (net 13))
 (segment (start 142.600073 141.46003) (end 141.890387 137.381197) (width 0.25) (layer "F.Cu") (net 16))
 (segment (start 143.890759 140.493835) (end 143.768774 136.35552) (width 0.25) (layer "F.Cu") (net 10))
 (segment (start 145.30581 139.721158) (end 145.774011 135.607605) (width 0.25) (layer "F.Cu") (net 11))
 (segment (start 146.816421 139.157729) (end 147.865277 135.152678) (width 0.25) (layer "F.Cu") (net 7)))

